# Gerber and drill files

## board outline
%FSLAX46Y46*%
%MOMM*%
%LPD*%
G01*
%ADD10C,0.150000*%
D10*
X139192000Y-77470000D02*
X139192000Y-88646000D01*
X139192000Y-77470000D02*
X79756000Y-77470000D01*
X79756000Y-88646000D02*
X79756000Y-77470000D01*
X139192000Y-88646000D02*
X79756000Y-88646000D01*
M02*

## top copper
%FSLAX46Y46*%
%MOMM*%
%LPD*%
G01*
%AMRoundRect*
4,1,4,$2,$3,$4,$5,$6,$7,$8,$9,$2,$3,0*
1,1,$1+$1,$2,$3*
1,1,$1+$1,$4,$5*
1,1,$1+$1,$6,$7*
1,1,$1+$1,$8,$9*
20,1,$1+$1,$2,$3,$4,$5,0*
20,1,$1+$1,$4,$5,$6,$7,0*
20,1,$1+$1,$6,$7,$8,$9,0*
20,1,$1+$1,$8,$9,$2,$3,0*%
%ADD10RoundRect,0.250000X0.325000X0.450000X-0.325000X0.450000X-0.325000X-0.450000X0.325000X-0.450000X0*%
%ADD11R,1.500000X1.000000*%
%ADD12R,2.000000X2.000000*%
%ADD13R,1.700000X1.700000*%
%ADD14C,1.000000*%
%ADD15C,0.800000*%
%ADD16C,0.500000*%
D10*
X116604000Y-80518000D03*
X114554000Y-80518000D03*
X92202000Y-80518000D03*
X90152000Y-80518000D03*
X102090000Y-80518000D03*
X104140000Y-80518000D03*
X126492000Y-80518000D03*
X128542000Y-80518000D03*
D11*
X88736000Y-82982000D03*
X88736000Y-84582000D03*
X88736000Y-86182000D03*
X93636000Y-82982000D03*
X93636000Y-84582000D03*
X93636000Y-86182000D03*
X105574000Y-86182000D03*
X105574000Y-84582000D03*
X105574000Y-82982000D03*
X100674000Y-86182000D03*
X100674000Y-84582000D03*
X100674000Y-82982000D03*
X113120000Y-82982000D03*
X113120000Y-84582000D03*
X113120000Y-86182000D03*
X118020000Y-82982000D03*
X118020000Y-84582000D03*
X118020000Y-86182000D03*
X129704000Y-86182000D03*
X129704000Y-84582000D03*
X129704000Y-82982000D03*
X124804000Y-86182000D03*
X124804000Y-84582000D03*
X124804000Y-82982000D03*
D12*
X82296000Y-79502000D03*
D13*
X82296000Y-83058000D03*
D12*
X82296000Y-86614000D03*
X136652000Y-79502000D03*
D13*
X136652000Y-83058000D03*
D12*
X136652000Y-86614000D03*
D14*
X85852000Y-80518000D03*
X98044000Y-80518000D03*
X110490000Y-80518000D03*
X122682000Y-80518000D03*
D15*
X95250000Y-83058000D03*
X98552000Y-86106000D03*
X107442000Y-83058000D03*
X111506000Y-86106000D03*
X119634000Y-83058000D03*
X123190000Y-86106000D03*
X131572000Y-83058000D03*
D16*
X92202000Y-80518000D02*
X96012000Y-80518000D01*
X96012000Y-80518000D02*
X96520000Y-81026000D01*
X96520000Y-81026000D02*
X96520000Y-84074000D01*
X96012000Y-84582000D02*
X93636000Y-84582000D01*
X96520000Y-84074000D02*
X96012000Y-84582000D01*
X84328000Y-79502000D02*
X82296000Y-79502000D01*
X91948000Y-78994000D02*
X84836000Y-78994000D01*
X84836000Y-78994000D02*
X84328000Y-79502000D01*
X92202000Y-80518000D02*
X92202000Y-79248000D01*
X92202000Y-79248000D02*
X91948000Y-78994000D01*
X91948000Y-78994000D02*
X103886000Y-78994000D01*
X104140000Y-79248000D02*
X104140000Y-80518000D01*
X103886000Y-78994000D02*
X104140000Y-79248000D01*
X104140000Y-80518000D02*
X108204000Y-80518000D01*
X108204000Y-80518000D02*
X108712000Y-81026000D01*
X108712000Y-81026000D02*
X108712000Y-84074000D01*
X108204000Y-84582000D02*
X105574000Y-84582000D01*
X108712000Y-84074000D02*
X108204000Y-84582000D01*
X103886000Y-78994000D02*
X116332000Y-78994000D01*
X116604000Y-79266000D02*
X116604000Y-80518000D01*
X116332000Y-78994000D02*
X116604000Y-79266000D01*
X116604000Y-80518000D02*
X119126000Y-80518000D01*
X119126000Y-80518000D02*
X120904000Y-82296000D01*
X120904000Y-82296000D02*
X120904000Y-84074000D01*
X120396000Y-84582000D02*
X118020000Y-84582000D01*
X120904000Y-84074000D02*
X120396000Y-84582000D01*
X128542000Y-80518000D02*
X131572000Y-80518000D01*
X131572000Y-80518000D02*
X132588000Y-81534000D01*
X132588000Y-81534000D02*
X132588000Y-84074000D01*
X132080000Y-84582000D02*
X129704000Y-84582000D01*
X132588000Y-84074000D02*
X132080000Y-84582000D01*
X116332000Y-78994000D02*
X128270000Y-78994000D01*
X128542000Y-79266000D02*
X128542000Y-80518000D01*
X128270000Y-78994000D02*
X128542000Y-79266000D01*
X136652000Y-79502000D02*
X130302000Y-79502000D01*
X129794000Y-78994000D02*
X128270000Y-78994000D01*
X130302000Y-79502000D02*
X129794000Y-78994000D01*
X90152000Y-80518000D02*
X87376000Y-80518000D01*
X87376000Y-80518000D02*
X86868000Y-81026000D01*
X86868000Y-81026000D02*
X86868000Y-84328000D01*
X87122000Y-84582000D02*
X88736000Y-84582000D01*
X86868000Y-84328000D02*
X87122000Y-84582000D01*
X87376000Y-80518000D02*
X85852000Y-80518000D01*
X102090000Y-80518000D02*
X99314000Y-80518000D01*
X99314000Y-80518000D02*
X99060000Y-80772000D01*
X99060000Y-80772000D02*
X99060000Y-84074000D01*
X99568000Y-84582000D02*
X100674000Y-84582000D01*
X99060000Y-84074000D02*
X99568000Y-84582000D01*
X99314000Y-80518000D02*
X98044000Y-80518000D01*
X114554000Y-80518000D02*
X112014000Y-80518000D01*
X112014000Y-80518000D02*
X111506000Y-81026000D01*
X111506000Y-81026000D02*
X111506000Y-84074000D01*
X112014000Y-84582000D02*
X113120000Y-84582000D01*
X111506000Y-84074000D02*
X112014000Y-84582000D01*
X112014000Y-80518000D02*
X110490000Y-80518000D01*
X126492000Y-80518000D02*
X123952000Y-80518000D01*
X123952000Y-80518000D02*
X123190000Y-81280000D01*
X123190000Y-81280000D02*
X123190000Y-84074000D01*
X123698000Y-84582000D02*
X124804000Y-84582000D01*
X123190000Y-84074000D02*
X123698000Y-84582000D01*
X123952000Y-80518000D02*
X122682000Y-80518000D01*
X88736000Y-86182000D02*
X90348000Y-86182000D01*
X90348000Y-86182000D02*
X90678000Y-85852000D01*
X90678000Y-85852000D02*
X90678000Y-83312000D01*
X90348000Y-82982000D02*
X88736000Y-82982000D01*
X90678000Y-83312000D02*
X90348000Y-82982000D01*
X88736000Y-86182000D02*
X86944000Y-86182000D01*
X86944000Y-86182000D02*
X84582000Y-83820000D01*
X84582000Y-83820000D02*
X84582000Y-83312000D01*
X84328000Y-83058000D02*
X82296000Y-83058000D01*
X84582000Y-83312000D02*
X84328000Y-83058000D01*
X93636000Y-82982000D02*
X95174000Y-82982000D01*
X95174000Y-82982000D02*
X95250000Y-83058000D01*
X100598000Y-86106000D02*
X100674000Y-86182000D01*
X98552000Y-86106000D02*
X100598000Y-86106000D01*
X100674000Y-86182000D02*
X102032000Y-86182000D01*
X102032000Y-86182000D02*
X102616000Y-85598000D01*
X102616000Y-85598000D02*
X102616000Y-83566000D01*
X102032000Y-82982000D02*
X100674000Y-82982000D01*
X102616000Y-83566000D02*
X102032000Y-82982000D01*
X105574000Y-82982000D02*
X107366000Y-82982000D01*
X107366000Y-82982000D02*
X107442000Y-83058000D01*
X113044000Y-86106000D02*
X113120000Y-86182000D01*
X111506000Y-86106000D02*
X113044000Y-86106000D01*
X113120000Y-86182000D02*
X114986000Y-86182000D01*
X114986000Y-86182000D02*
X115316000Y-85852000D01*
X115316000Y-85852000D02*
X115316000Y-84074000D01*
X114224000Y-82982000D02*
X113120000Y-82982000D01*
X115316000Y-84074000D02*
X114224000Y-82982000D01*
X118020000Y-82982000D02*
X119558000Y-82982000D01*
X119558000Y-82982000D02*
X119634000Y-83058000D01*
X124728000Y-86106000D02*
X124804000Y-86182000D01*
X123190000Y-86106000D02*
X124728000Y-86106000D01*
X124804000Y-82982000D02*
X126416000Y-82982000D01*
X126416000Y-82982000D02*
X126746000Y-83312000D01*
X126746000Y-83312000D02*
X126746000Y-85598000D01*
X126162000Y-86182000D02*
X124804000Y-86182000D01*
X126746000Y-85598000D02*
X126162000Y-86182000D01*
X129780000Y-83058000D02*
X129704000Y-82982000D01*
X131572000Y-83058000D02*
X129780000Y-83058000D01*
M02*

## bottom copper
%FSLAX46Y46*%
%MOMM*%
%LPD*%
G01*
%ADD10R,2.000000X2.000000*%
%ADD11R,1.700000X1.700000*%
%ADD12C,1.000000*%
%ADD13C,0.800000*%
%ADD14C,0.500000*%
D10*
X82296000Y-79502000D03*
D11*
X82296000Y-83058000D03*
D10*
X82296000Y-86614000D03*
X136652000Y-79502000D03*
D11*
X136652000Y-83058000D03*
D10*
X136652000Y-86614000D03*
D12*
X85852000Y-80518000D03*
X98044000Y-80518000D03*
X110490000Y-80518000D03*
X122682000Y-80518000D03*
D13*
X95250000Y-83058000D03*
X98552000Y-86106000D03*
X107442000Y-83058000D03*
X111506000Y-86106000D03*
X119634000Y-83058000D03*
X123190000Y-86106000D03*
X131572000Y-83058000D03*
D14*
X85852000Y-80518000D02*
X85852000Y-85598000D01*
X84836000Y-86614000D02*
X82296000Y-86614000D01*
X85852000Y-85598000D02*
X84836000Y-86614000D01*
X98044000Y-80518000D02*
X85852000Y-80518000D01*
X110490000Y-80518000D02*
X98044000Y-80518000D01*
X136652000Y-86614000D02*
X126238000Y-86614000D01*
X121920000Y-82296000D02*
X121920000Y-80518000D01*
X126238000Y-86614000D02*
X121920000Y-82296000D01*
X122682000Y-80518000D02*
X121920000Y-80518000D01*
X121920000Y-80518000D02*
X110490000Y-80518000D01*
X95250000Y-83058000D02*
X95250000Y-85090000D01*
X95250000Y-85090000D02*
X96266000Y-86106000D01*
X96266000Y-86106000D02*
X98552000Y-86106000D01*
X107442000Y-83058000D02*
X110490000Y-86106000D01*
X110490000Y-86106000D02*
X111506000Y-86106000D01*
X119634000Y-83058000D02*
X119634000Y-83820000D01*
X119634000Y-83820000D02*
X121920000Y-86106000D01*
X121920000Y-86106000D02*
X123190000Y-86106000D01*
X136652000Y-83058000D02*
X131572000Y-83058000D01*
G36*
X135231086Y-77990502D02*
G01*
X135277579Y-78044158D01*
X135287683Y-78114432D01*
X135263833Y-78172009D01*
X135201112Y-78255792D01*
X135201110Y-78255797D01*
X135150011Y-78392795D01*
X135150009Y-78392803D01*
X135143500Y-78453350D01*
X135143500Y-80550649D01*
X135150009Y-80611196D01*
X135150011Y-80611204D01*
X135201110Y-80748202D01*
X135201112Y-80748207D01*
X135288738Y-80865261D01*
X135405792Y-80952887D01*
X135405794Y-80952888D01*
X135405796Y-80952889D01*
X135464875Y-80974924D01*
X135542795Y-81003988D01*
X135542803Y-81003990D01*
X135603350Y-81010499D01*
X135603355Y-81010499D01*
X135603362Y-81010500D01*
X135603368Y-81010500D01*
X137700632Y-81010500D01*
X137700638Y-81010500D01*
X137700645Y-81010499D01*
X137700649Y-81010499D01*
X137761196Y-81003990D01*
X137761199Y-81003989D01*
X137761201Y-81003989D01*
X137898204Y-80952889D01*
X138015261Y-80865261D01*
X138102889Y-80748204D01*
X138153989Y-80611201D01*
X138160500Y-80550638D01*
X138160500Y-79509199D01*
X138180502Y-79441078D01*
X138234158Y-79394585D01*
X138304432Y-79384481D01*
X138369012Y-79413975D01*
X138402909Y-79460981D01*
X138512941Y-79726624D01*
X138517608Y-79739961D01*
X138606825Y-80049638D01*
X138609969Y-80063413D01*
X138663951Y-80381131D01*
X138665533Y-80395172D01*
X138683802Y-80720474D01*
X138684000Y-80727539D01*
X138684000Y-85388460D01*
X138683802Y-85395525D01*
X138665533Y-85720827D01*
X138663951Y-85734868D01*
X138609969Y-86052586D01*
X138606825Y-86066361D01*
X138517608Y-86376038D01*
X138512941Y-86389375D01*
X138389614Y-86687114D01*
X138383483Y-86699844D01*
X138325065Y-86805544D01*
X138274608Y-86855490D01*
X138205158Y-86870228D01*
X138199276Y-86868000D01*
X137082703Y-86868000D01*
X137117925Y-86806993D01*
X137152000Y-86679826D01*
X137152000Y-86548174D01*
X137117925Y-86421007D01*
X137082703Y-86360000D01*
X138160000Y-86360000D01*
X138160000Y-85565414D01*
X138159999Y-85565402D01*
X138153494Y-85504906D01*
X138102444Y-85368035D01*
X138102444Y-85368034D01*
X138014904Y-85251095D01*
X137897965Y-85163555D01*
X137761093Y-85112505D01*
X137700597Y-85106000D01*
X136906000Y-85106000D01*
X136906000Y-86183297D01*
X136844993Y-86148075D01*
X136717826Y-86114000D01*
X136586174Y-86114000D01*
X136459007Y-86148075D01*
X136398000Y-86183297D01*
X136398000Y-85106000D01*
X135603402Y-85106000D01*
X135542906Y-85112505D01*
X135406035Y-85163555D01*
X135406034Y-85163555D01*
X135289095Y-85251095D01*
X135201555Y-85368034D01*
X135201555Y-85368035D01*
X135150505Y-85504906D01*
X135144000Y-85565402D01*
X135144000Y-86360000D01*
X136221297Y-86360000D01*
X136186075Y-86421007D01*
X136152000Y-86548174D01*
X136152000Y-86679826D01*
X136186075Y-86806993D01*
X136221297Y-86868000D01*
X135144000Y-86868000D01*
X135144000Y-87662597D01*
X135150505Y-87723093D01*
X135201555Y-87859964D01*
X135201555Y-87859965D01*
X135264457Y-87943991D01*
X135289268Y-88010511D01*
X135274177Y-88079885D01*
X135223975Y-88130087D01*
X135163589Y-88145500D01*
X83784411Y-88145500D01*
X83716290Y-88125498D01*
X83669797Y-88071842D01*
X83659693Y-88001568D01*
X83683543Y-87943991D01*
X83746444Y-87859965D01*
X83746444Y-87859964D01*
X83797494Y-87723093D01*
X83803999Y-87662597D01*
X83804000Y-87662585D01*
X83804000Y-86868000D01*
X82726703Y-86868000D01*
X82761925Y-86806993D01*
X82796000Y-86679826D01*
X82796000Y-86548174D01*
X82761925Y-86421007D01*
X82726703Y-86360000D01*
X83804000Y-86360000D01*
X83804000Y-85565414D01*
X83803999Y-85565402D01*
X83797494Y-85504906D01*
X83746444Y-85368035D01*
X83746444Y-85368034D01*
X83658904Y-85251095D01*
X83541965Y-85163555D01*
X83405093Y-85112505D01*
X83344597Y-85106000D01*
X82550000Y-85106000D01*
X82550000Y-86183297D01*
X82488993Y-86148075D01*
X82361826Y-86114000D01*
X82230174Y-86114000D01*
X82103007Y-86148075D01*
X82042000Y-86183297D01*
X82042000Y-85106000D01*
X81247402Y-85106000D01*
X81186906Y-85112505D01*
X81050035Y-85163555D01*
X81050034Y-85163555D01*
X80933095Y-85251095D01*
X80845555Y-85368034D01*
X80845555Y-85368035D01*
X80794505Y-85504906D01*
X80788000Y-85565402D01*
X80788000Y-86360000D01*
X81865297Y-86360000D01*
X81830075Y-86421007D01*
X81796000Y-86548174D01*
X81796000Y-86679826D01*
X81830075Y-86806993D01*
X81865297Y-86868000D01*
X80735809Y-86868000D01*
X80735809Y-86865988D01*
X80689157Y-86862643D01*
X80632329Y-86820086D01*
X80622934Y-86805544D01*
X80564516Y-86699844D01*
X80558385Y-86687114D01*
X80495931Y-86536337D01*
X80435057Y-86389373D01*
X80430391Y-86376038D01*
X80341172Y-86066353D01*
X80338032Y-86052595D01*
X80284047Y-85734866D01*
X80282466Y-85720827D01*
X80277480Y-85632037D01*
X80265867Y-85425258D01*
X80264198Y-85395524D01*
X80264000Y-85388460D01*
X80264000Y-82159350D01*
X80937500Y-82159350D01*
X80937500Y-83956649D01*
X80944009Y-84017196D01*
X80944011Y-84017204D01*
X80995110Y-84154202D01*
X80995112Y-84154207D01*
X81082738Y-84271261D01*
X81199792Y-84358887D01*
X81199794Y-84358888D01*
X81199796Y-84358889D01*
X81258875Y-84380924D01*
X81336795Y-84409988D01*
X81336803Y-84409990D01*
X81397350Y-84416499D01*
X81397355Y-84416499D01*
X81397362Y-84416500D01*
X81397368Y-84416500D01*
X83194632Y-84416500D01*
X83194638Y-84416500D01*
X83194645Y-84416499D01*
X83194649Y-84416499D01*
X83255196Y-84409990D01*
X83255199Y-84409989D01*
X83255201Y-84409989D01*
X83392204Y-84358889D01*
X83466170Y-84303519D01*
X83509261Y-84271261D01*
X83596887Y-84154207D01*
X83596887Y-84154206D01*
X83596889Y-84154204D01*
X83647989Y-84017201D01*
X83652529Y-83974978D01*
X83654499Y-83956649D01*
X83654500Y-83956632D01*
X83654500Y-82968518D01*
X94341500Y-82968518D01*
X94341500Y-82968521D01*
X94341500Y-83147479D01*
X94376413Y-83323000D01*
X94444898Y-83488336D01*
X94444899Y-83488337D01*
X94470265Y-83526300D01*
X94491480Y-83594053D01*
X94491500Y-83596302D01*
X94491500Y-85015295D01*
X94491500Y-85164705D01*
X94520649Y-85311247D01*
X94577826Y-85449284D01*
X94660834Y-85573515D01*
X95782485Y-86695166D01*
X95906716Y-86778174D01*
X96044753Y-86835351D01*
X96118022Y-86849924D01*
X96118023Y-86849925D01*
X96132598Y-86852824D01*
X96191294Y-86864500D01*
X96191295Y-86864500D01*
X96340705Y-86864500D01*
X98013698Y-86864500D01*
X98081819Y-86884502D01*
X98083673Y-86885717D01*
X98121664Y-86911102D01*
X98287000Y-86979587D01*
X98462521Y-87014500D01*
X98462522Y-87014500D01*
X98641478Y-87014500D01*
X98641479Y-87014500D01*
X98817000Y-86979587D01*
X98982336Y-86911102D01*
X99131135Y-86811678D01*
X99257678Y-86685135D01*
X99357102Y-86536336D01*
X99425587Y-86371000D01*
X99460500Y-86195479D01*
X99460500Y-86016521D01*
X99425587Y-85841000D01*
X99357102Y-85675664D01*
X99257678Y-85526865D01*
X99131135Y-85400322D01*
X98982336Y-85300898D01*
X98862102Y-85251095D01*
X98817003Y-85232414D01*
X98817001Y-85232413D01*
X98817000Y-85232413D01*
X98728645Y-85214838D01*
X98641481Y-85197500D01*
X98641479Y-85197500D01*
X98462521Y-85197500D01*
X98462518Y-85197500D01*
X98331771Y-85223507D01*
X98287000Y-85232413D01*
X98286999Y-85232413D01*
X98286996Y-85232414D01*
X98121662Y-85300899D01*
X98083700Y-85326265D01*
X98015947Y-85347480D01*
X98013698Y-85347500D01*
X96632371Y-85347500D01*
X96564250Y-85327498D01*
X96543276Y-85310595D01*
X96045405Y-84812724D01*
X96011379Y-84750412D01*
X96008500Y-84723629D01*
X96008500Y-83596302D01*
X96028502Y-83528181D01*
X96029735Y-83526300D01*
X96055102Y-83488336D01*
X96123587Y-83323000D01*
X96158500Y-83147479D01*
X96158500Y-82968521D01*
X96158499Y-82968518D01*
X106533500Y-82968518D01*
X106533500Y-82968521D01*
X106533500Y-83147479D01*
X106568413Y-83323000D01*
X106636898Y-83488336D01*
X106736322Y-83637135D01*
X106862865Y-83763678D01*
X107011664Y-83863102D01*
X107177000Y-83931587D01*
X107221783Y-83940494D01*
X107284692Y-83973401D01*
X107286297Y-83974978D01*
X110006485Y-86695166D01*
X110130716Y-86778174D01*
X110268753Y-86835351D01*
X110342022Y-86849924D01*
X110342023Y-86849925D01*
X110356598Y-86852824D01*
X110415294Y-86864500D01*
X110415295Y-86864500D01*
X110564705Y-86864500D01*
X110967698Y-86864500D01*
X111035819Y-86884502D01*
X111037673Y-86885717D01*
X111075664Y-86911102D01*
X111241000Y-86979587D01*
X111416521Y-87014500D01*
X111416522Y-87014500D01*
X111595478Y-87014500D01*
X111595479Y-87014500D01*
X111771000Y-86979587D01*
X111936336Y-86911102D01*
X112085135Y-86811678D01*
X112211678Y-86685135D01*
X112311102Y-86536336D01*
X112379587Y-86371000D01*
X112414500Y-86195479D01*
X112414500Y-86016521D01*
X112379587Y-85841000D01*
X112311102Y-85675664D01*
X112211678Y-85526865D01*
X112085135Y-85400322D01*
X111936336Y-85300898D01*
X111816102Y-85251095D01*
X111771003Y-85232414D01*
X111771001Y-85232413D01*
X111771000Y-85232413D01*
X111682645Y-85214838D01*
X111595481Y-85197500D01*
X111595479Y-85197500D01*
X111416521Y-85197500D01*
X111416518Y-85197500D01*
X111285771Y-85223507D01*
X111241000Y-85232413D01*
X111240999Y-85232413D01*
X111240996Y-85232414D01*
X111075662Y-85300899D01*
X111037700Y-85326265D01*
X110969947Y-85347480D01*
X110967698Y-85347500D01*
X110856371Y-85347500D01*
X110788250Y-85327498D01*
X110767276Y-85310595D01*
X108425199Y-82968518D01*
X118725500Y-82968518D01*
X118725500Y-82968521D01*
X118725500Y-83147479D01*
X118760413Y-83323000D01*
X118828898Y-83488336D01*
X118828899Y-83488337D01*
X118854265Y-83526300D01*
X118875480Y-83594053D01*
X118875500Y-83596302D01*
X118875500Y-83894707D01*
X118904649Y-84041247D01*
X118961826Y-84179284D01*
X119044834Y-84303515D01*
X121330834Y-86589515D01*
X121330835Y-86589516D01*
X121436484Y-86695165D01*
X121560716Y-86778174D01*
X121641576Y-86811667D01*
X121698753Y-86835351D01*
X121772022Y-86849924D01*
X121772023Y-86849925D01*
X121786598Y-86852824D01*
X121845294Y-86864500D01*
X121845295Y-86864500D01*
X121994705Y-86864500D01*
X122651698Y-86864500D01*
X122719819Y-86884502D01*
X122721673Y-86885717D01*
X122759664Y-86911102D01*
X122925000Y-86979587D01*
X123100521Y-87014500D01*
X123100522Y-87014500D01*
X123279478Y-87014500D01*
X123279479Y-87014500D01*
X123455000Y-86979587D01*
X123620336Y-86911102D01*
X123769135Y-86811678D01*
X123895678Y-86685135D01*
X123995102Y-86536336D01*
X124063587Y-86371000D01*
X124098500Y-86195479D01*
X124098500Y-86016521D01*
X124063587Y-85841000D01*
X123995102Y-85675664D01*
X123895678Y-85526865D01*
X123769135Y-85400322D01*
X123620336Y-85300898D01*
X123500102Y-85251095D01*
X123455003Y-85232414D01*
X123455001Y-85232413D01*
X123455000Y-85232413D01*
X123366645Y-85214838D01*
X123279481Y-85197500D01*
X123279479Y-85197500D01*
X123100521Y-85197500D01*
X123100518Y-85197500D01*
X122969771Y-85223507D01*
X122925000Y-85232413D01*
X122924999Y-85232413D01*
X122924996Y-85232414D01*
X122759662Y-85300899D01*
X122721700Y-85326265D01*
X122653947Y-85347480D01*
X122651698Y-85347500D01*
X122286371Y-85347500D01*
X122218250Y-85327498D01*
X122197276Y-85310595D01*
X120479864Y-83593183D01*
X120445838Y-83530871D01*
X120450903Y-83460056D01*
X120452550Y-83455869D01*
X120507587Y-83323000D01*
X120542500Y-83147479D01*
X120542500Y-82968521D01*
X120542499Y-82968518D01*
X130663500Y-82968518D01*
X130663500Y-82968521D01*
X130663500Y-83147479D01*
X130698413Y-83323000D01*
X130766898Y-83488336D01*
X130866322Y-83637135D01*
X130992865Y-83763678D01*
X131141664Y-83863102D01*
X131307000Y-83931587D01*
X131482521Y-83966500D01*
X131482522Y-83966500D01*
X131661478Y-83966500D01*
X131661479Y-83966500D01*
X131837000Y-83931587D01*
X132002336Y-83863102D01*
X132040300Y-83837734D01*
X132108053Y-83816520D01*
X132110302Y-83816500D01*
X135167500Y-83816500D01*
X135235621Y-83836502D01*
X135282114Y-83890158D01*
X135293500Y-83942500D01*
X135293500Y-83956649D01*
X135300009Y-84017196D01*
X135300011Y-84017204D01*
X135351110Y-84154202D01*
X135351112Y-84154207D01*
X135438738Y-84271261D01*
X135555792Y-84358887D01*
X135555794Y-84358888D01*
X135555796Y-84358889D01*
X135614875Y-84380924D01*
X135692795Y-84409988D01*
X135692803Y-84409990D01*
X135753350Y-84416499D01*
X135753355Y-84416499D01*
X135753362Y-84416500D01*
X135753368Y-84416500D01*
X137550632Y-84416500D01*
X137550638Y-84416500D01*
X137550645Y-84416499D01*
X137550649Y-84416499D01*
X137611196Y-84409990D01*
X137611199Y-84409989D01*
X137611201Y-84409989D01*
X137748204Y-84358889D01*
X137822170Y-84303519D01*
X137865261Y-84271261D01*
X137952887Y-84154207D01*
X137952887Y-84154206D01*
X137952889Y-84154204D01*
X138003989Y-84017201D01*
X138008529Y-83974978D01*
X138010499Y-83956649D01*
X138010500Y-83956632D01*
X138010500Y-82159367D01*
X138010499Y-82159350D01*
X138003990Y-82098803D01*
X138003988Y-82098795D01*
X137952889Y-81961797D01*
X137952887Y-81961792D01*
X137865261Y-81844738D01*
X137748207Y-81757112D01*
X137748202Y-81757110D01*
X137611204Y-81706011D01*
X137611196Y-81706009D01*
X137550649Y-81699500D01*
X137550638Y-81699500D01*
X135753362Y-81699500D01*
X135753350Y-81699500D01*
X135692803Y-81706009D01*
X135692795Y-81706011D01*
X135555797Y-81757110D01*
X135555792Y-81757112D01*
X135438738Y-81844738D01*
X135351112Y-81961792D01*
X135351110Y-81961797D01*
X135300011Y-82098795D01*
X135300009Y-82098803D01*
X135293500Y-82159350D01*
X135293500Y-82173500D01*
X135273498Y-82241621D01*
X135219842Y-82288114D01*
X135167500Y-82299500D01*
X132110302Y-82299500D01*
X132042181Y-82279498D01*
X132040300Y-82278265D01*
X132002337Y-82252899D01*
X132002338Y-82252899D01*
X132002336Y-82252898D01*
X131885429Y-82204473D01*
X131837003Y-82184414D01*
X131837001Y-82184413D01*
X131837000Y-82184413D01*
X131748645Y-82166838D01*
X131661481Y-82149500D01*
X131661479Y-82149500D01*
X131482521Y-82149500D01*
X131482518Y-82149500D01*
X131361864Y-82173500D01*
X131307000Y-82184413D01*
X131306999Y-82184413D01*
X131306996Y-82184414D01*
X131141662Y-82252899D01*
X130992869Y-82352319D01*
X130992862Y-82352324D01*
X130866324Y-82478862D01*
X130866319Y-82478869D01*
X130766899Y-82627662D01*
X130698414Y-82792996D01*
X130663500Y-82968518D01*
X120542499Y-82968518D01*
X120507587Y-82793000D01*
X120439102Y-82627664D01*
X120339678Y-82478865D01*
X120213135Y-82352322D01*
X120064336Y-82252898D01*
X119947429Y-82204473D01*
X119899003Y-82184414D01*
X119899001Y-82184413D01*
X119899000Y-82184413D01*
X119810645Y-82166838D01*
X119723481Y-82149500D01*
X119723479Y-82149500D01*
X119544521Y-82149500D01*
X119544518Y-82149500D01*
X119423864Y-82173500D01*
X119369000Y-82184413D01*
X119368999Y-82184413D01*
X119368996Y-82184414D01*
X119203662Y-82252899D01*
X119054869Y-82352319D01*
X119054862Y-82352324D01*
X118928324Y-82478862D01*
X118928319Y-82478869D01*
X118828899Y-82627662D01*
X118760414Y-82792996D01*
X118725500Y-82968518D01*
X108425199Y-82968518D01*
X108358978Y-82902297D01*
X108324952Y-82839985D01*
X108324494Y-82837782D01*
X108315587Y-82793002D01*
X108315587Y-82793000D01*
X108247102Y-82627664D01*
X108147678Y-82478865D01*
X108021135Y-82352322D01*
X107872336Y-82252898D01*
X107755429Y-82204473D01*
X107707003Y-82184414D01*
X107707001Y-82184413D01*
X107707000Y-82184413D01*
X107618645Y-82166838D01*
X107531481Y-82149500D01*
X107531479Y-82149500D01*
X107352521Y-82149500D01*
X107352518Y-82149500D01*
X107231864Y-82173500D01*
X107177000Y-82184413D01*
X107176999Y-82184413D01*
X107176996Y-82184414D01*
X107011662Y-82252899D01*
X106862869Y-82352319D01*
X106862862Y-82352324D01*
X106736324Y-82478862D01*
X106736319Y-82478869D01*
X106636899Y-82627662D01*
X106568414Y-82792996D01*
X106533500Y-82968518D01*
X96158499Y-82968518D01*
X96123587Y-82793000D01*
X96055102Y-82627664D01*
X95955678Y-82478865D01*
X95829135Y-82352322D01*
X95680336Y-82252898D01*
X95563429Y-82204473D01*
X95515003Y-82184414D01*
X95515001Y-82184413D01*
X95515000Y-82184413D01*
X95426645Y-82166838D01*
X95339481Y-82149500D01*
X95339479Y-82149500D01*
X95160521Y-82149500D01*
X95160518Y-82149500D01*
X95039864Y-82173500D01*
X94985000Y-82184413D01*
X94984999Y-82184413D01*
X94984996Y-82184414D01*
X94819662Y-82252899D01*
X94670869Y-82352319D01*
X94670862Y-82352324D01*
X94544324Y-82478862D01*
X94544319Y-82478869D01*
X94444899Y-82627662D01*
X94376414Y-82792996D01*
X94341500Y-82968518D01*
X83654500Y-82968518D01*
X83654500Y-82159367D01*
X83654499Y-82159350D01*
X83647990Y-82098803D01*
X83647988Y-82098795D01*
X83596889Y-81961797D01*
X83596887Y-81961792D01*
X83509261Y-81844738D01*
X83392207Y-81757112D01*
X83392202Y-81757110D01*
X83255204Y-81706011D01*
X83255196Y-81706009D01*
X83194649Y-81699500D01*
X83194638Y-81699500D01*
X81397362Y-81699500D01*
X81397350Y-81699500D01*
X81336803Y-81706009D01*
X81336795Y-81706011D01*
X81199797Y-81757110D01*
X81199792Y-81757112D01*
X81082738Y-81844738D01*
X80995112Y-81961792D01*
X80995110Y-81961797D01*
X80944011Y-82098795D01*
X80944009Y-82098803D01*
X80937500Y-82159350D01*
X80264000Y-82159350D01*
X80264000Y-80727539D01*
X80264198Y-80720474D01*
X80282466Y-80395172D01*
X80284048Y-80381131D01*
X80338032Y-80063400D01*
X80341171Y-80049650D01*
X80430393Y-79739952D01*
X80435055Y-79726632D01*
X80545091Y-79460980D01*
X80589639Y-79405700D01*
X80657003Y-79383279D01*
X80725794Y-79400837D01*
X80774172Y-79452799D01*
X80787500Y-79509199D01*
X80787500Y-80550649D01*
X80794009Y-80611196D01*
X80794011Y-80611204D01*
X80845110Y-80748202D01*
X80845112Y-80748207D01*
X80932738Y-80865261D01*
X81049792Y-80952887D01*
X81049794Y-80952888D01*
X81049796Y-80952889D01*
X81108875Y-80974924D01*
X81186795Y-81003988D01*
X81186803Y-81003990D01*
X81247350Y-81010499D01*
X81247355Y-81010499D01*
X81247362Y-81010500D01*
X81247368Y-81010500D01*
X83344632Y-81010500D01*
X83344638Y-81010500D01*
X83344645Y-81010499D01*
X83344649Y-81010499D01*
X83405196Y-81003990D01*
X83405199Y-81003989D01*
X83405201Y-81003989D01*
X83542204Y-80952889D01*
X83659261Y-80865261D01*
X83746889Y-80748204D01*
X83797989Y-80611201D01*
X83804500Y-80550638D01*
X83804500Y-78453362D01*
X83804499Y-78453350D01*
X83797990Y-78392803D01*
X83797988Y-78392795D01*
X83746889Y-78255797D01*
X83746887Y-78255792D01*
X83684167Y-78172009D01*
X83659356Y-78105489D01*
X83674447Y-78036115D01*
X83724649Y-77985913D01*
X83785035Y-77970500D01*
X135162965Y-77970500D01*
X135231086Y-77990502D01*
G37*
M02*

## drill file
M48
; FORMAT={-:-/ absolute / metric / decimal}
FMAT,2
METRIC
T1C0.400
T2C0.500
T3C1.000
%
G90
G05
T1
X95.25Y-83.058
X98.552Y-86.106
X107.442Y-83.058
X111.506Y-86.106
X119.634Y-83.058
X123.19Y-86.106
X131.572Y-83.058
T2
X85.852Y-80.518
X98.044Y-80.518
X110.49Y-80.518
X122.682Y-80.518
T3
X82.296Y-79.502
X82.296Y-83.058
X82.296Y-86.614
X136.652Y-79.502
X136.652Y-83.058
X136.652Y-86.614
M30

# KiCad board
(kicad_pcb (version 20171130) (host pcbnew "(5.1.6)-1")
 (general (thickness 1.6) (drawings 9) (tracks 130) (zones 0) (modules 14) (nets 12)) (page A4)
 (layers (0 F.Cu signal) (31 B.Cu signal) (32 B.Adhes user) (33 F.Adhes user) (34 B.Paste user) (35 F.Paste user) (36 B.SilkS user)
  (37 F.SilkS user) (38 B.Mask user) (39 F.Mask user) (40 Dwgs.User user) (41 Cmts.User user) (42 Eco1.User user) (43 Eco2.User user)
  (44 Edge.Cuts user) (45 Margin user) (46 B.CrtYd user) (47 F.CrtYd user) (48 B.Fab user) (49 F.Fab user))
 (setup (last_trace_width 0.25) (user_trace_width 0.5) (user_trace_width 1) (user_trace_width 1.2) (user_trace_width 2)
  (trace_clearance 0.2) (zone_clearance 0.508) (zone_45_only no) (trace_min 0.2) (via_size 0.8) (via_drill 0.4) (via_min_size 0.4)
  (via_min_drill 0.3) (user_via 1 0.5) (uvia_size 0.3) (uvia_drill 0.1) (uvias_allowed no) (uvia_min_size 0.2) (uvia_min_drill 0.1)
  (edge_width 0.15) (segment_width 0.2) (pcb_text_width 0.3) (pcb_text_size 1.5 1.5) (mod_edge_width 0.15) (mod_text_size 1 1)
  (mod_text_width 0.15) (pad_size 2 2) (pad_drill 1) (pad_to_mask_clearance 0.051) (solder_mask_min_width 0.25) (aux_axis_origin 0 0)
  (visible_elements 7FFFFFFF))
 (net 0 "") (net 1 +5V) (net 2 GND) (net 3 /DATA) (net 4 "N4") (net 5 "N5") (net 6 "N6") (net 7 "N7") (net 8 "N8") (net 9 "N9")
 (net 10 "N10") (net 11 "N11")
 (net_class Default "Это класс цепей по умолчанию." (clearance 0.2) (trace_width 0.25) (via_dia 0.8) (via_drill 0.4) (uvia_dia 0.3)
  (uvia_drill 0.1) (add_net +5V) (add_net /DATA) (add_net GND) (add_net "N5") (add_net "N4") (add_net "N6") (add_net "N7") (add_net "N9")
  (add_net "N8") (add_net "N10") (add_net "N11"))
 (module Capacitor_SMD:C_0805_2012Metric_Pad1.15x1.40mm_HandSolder (layer F.Cu) (at 115.579 80.518 180)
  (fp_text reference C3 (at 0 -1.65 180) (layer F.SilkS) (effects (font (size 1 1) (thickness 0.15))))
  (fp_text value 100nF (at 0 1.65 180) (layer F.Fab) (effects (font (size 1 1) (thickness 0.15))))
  (pad 1 smd roundrect (at -1.025 0 180) (size 1.15 1.4) (layers F.Cu F.Paste F.Mask) (roundrect_rratio 0.217391) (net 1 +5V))
  (pad 2 smd roundrect (at 1.025 0 180) (size 1.15 1.4) (layers F.Cu F.Paste F.Mask) (roundrect_rratio 0.217391) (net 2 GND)))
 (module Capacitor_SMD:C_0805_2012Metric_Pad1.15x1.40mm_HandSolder (layer F.Cu) (at 91.177 80.518 180)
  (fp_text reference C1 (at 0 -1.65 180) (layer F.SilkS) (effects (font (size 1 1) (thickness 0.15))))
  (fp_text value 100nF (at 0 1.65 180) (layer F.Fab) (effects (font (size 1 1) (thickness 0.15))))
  (pad 1 smd roundrect (at -1.025 0 180) (size 1.15 1.4) (layers F.Cu F.Paste F.Mask) (roundrect_rratio 0.217391) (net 1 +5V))
  (pad 2 smd roundrect (at 1.025 0 180) (size 1.15 1.4) (layers F.Cu F.Paste F.Mask) (roundrect_rratio 0.217391) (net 2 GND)))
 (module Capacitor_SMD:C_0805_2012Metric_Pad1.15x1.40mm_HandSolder (layer F.Cu) (at 103.115 80.518 180)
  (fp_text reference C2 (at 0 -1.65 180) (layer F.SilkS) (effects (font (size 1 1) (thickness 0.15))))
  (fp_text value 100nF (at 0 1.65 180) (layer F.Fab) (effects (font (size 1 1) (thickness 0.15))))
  (pad 2 smd roundrect (at 1.025 0 180) (size 1.15 1.4) (layers F.Cu F.Paste F.Mask) (roundrect_rratio 0.217391) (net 2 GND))
  (pad 1 smd roundrect (at -1.025 0 180) (size 1.15 1.4) (layers F.Cu F.Paste F.Mask) (roundrect_rratio 0.217391) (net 1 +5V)))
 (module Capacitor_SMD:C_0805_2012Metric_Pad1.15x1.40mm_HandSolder (layer F.Cu) (at 127.517 80.518 180)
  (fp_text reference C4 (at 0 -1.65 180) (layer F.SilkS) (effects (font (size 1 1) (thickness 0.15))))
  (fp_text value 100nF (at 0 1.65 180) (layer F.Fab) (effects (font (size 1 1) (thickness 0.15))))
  (pad 2 smd roundrect (at 1.025 0 180) (size 1.15 1.4) (layers F.Cu F.Paste F.Mask) (roundrect_rratio 0.217391) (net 2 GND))
  (pad 1 smd roundrect (at -1.025 0 180) (size 1.15 1.4) (layers F.Cu F.Paste F.Mask) (roundrect_rratio 0.217391) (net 1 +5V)))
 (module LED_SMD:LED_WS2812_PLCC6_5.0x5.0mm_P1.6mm (layer F.Cu) (at 91.186 84.582 180)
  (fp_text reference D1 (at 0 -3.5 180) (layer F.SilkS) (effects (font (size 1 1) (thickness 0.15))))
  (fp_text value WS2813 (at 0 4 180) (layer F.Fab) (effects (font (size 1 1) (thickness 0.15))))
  (pad 4 smd rect (at 2.45 1.6 180) (size 1.5 1) (layers F.Cu F.Paste F.Mask) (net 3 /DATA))
  (pad 5 smd rect (at 2.45 0 180) (size 1.5 1) (layers F.Cu F.Paste F.Mask) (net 2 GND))
  (pad 6 smd rect (at 2.45 -1.6 180) (size 1.5 1) (layers F.Cu F.Paste F.Mask) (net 3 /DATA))
  (pad 3 smd rect (at -2.45 1.6 180) (size 1.5 1) (layers F.Cu F.Paste F.Mask) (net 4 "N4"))
  (pad 2 smd rect (at -2.45 0 180) (size 1.5 1) (layers F.Cu F.Paste F.Mask) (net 1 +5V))
  (pad 1 smd rect (at -2.45 -1.6 180) (size 1.5 1) (layers F.Cu F.Paste F.Mask) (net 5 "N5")))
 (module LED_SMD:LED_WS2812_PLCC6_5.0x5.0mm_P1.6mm (layer F.Cu) (at 103.124 84.582 180)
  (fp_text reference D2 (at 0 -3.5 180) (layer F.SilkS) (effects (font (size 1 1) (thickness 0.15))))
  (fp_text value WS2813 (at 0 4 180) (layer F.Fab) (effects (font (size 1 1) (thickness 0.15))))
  (pad 1 smd rect (at -2.45 -1.6 180) (size 1.5 1) (layers F.Cu F.Paste F.Mask) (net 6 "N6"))
  (pad 2 smd rect (at -2.45 0 180) (size 1.5 1) (layers F.Cu F.Paste F.Mask) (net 1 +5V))
  (pad 3 smd rect (at -2.45 1.6 180) (size 1.5 1) (layers F.Cu F.Paste F.Mask) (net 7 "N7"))
  (pad 6 smd rect (at 2.45 -1.6 180) (size 1.5 1) (layers F.Cu F.Paste F.Mask) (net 4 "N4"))
  (pad 5 smd rect (at 2.45 0 180) (size 1.5 1) (layers F.Cu F.Paste F.Mask) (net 2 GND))
  (pad 4 smd rect (at 2.45 1.6 180) (size 1.5 1) (layers F.Cu F.Paste F.Mask) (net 4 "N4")))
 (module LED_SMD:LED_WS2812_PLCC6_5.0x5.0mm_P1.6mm (layer F.Cu) (at 115.57 84.582 180)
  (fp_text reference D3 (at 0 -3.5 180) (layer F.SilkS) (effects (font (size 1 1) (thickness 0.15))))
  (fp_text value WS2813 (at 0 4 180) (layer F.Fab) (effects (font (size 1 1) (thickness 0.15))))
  (pad 4 smd rect (at 2.45 1.6 180) (size 1.5 1) (layers F.Cu F.Paste F.Mask) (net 7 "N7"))
  (pad 5 smd rect (at 2.45 0 180) (size 1.5 1) (layers F.Cu F.Paste F.Mask) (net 2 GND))
  (pad 6 smd rect (at 2.45 -1.6 180) (size 1.5 1) (layers F.Cu F.Paste F.Mask) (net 7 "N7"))
  (pad 3 smd rect (at -2.45 1.6 180) (size 1.5 1) (layers F.Cu F.Paste F.Mask) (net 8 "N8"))
  (pad 2 smd rect (at -2.45 0 180) (size 1.5 1) (layers F.Cu F.Paste F.Mask) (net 1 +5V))
  (pad 1 smd rect (at -2.45 -1.6 180) (size 1.5 1) (layers F.Cu F.Paste F.Mask) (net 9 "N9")))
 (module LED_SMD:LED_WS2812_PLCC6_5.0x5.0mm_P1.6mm (layer F.Cu) (at 127.254 84.582 180)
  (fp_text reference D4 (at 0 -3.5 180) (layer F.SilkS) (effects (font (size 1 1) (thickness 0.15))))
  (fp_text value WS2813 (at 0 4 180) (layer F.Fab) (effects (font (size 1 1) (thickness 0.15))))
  (pad 1 smd rect (at -2.45 -1.6 180) (size 1.5 1) (layers F.Cu F.Paste F.Mask) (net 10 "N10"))
  (pad 2 smd rect (at -2.45 0 180) (size 1.5 1) (layers F.Cu F.Paste F.Mask) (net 1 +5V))
  (pad 3 smd rect (at -2.45 1.6 180) (size 1.5 1) (layers F.Cu F.Paste F.Mask) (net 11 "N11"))
  (pad 6 smd rect (at 2.45 -1.6 180) (size 1.5 1) (layers F.Cu F.Paste F.Mask) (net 8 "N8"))
  (pad 5 smd rect (at 2.45 0 180) (size 1.5 1) (layers F.Cu F.Paste F.Mask) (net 2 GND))
  (pad 4 smd rect (at 2.45 1.6 180) (size 1.5 1) (layers F.Cu F.Paste F.Mask) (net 8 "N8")))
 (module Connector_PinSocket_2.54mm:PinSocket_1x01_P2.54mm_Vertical (layer F.Cu) (at 82.296 79.502)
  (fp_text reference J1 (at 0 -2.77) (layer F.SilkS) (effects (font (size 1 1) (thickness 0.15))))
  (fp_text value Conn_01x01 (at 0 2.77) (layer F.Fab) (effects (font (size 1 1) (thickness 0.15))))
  (pad 1 thru_hole rect (at 0 0) (size 2 2) (drill 1) (layers *.Cu *.Mask) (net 1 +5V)))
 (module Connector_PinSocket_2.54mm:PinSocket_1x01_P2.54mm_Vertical (layer F.Cu) (at 82.296 83.058)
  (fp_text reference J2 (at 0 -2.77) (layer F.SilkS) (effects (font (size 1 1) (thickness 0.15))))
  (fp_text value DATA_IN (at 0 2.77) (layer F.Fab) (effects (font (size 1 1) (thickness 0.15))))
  (pad 1 thru_hole rect (at 0 0) (size 1.7 1.7) (drill 1) (layers *.Cu *.Mask) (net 3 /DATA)))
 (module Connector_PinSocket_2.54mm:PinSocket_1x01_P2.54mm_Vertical (layer F.Cu) (at 82.296 86.614)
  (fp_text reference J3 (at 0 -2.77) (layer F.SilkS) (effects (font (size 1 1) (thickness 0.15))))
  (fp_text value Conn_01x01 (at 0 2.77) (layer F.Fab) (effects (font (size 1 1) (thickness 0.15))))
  (pad 1 thru_hole rect (at 0 0) (size 2 2) (drill 1) (layers *.Cu *.Mask) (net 2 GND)))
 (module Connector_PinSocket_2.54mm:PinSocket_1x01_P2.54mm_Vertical (layer F.Cu) (at 136.652 79.502)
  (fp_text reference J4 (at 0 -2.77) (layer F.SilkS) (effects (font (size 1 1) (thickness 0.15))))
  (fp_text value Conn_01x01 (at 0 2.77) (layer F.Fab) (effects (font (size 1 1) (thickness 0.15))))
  (pad 1 thru_hole rect (at 0 0) (size 2 2) (drill 1) (layers *.Cu *.Mask) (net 1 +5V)))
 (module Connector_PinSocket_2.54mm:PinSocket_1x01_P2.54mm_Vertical (layer F.Cu) (at 136.652 83.058)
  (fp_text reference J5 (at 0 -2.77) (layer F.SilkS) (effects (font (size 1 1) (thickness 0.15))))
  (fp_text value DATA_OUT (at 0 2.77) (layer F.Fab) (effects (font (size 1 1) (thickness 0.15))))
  (pad 1 thru_hole rect (at 0 0) (size 1.7 1.7) (drill 1) (layers *.Cu *.Mask) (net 11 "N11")))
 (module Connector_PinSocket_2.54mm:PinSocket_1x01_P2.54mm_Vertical (layer F.Cu) (at 136.652 86.614)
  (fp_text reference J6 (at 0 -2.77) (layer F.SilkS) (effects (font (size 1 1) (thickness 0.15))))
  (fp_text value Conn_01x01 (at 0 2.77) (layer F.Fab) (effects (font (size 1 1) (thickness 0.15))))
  (pad 1 thru_hole rect (at 0 0) (size 2 2) (drill 1) (layers *.Cu *.Mask) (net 2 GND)))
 (gr_line (start 139.192 77.47) (end 139.192 88.646) (layer Edge.Cuts) (width 0.15))
 (gr_line (start 139.192 77.47) (end 79.756 77.47) (layer Edge.Cuts) (width 0.15))
 (gr_line (start 79.756 88.646) (end 79.756 77.47) (layer Edge.Cuts) (width 0.15))
 (gr_line (start 139.192 88.646) (end 79.756 88.646) (layer Edge.Cuts) (width 0.15))
 (segment (start 92.202 80.518) (end 96.012 80.518) (width 0.5) (layer F.Cu) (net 1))
 (segment (start 96.012 80.518) (end 96.52 81.026) (width 0.5) (layer F.Cu) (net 1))
 (segment (start 96.52 81.026) (end 96.52 84.074) (width 0.5) (layer F.Cu) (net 1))
 (segment (start 96.012 84.582) (end 93.636 84.582) (width 0.5) (layer F.Cu) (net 1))
 (segment (start 96.52 84.074) (end 96.012 84.582) (width 0.5) (layer F.Cu) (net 1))
 (segment (start 84.328 79.502) (end 82.296 79.502) (width 0.5) (layer F.Cu) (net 1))
 (segment (start 91.948 78.994) (end 84.836 78.994) (width 0.5) (layer F.Cu) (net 1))
 (segment (start 84.836 78.994) (end 84.328 79.502) (width 0.5) (layer F.Cu) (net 1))
 (segment (start 92.202 80.518) (end 92.202 79.248) (width 0.5) (layer F.Cu) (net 1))
 (segment (start 92.202 79.248) (end 91.948 78.994) (width 0.5) (layer F.Cu) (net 1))
 (segment (start 91.948 78.994) (end 103.886 78.994) (width 0.5) (layer F.Cu) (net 1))
 (segment (start 104.14 79.248) (end 104.14 80.518) (width 0.5) (layer F.Cu) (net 1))
 (segment (start 103.886 78.994) (end 104.14 79.248) (width 0.5) (layer F.Cu) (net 1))
 (segment (start 104.14 80.518) (end 108.204 80.518) (width 0.5) (layer F.Cu) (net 1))
 (segment (start 108.204 80.518) (end 108.712 81.026) (width 0.5) (layer F.Cu) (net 1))
 (segment (start 108.712 81.026) (end 108.712 84.074) (width 0.5) (layer F.Cu) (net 1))
 (segment (start 108.204 84.582) (end 105.574 84.582) (width 0.5) (layer F.Cu) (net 1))
 (segment (start 108.712 84.074) (end 108.204 84.582) (width 0.5) (layer F.Cu) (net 1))
 (segment (start 103.886 78.994) (end 116.332 78.994) (width 0.5) (layer F.Cu) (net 1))
 (segment (start 116.604 79.266) (end 116.604 80.518) (width 0.5) (layer F.Cu) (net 1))
 (segment (start 116.332 78.994) (end 116.604 79.266) (width 0.5) (layer F.Cu) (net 1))
 (segment (start 116.604 80.518) (end 119.126 80.518) (width 0.5) (layer F.Cu) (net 1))
 (segment (start 119.126 80.518) (end 120.904 82.296) (width 0.5) (layer F.Cu) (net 1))
 (segment (start 120.904 82.296) (end 120.904 84.074) (width 0.5) (layer F.Cu) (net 1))
 (segment (start 120.396 84.582) (end 118.02 84.582) (width 0.5) (layer F.Cu) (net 1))
 (segment (start 120.904 84.074) (end 120.396 84.582) (width 0.5) (layer F.Cu) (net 1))
 (segment (start 128.542 80.518) (end 131.572 80.518) (width 0.5) (layer F.Cu) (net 1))
 (segment (start 131.572 80.518) (end 132.588 81.534) (width 0.5) (layer F.Cu) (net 1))
 (segment (start 132.588 81.534) (end 132.588 84.074) (width 0.5) (layer F.Cu) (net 1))
 (segment (start 132.08 84.582) (end 129.704 84.582) (width 0.5) (layer F.Cu) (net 1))
 (segment (start 132.588 84.074) (end 132.08 84.582) (width 0.5) (layer F.Cu) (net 1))
 (segment (start 116.332 78.994) (end 128.27 78.994) (width 0.5) (layer F.Cu) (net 1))
 (segment (start 128.542 79.266) (end 128.542 80.518) (width 0.5) (layer F.Cu) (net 1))
 (segment (start 128.27 78.994) (end 128.542 79.266) (width 0.5) (layer F.Cu) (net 1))
 (segment (start 136.652 79.502) (end 130.302 79.502) (width 0.5) (layer F.Cu) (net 1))
 (segment (start 129.794 78.994) (end 128.27 78.994) (width 0.5) (layer F.Cu) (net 1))
 (segment (start 130.302 79.502) (end 129.794 78.994) (width 0.5) (layer F.Cu) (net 1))
 (segment (start 90.152 80.518) (end 87.376 80.518) (width 0.5) (layer F.Cu) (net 2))
 (segment (start 87.376 80.518) (end 86.868 81.026) (width 0.5) (layer F.Cu) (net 2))
 (segment (start 86.868 81.026) (end 86.868 84.328) (width 0.5) (layer F.Cu) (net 2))
 (segment (start 87.122 84.582) (end 88.736 84.582) (width 0.5) (layer F.Cu) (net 2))
 (segment (start 86.868 84.328) (end 87.122 84.582) (width 0.5) (layer F.Cu) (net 2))
 (via (at 85.852 80.518) (size 1) (drill 0.5) (layers F.Cu B.Cu) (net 2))
 (segment (start 87.376 80.518) (end 85.852 80.518) (width 0.5) (layer F.Cu) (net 2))
 (segment (start 85.852 80.518) (end 85.852 85.598) (width 0.5) (layer B.Cu) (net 2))
 (segment (start 84.836 86.614) (end 82.296 86.614) (width 0.5) (layer B.Cu) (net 2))
 (segment (start 85.852 85.598) (end 84.836 86.614) (width 0.5) (layer B.Cu) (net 2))
 (segment (start 102.09 80.518) (end 99.314 80.518) (width 0.5) (layer F.Cu) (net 2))
 (segment (start 99.314 80.518) (end 99.06 80.772) (width 0.5) (layer F.Cu) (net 2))
 (segment (start 99.06 80.772) (end 99.06 84.074) (width 0.5) (layer F.Cu) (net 2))
 (segment (start 99.568 84.582) (end 100.674 84.582) (width 0.5) (layer F.Cu) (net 2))
 (segment (start 99.06 84.074) (end 99.568 84.582) (width 0.5) (layer F.Cu) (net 2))
 (via (at 98.044 80.518) (size 1) (drill 0.5) (layers F.Cu B.Cu) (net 2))
 (segment (start 99.314 80.518) (end 98.044 80.518) (width 0.5) (layer F.Cu) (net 2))
 (segment (start 98.044 80.518) (end 85.852 80.518) (width 0.5) (layer B.Cu) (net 2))
 (segment (start 114.554 80.518) (end 112.014 80.518) (width 0.5) (layer F.Cu) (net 2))
 (segment (start 112.014 80.518) (end 111.506 81.026) (width 0.5) (layer F.Cu) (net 2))
 (segment (start 111.506 81.026) (end 111.506 84.074) (width 0.5) (layer F.Cu) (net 2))
 (segment (start 112.014 84.582) (end 113.12 84.582) (width 0.5) (layer F.Cu) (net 2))
 (segment (start 111.506 84.074) (end 112.014 84.582) (width 0.5) (layer F.Cu) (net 2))
 (via (at 110.49 80.518) (size 1) (drill 0.5) (layers F.Cu B.Cu) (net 2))
 (segment (start 112.014 80.518) (end 110.49 80.518) (width 0.5) (layer F.Cu) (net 2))
 (segment (start 110.49 80.518) (end 98.044 80.518) (width 0.5) (layer B.Cu) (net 2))
 (segment (start 126.492 80.518) (end 123.952 80.518) (width 0.5) (layer F.Cu) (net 2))
 (segment (start 123.952 80.518) (end 123.19 81.28) (width 0.5) (layer F.Cu) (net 2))
 (segment (start 123.19 81.28) (end 123.19 84.074) (width 0.5) (layer F.Cu) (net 2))
 (segment (start 123.698 84.582) (end 124.804 84.582) (width 0.5) (layer F.Cu) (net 2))
 (segment (start 123.19 84.074) (end 123.698 84.582) (width 0.5) (layer F.Cu) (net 2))
 (via (at 122.682 80.518) (size 1) (drill 0.5) (layers F.Cu B.Cu) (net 2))
 (segment (start 123.952 80.518) (end 122.682 80.518) (width 0.5) (layer F.Cu) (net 2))
 (segment (start 136.652 86.614) (end 126.238 86.614) (width 0.5) (layer B.Cu) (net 2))
 (segment (start 121.92 82.296) (end 121.92 80.518) (width 0.5) (layer B.Cu) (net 2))
 (segment (start 126.238 86.614) (end 121.92 82.296) (width 0.5) (layer B.Cu) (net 2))
 (segment (start 122.682 80.518) (end 121.92 80.518) (width 0.5) (layer B.Cu) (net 2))
 (segment (start 121.92 80.518) (end 110.49 80.518) (width 0.5) (layer B.Cu) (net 2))
 (segment (start 88.736 86.182) (end 90.348 86.182) (width 0.5) (layer F.Cu) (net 3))
 (segment (start 90.348 86.182) (end 90.678 85.852) (width 0.5) (layer F.Cu) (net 3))
 (segment (start 90.678 85.852) (end 90.678 83.312) (width 0.5) (layer F.Cu) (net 3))
 (segment (start 90.348 82.982) (end 88.736 82.982) (width 0.5) (layer F.Cu) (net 3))
 (segment (start 90.678 83.312) (end 90.348 82.982) (width 0.5) (layer F.Cu) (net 3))
 (segment (start 88.736 86.182) (end 86.944 86.182) (width 0.5) (layer F.Cu) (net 3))
 (segment (start 86.944 86.182) (end 84.582 83.82) (width 0.5) (layer F.Cu) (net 3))
 (segment (start 84.582 83.82) (end 84.582 83.312) (width 0.5) (layer F.Cu) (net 3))
 (segment (start 84.328 83.058) (end 82.296 83.058) (width 0.5) (layer F.Cu) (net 3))
 (segment (start 84.582 83.312) (end 84.328 83.058) (width 0.5) (layer F.Cu) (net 3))
 (via (at 95.25 83.058) (size 0.8) (drill 0.4) (layers F.Cu B.Cu) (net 4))
 (segment (start 93.636 82.982) (end 95.174 82.982) (width 0.5) (layer F.Cu) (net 4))
 (segment (start 95.174 82.982) (end 95.25 83.058) (width 0.5) (layer F.Cu) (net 4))
 (segment (start 95.25 83.058) (end 95.25 85.09) (width 0.5) (layer B.Cu) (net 4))
 (via (at 98.552 86.106) (size 0.8) (drill 0.4) (layers F.Cu B.Cu) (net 4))
 (segment (start 95.25 85.09) (end 96.266 86.106) (width 0.5) (layer B.Cu) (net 4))
 (segment (start 96.266 86.106) (end 98.552 86.106) (width 0.5) (layer B.Cu) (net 4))
 (segment (start 100.598 86.106) (end 100.674 86.182) (width 0.5) (layer F.Cu) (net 4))
 (segment (start 98.552 86.106) (end 100.598 86.106) (width 0.5) (layer F.Cu) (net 4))
 (segment (start 100.674 86.182) (end 102.032 86.182) (width 0.5) (layer F.Cu) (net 4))
 (segment (start 102.032 86.182) (end 102.616 85.598) (width 0.5) (layer F.Cu) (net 4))
 (segment (start 102.616 85.598) (end 102.616 83.566) (width 0.5) (layer F.Cu) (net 4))
 (segment (start 102.032 82.982) (end 100.674 82.982) (width 0.5) (layer F.Cu) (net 4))
 (segment (start 102.616 83.566) (end 102.032 82.982) (width 0.5) (layer F.Cu) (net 4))
 (via (at 107.442 83.058) (size 0.8) (drill 0.4) (layers F.Cu B.Cu) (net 7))
 (segment (start 105.574 82.982) (end 107.366 82.982) (width 0.5) (layer F.Cu) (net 7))
 (segment (start 107.366 82.982) (end 107.442 83.058) (width 0.5) (layer F.Cu) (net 7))
 (via (at 111.506 86.106) (size 0.8) (drill 0.4) (layers F.Cu B.Cu) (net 7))
 (segment (start 107.442 83.058) (end 110.49 86.106) (width 0.5) (layer B.Cu) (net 7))
 (segment (start 110.49 86.106) (end 111.506 86.106) (width 0.5) (layer B.Cu) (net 7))
 (segment (start 113.044 86.106) (end 113.12 86.182) (width 0.5) (layer F.Cu) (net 7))
 (segment (start 111.506 86.106) (end 113.044 86.106) (width 0.5) (layer F.Cu) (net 7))
 (segment (start 113.12 86.182) (end 114.986 86.182) (width 0.5) (layer F.Cu) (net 7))
 (segment (start 114.986 86.182) (end 115.316 85.852) (width 0.5) (layer F.Cu) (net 7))
 (segment (start 115.316 85.852) (end 115.316 84.074) (width 0.5) (layer F.Cu) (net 7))
 (segment (start 114.224 82.982) (end 113.12 82.982) (width 0.5) (layer F.Cu) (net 7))
 (segment (start 115.316 84.074) (end 114.224 82.982) (width 0.5) (layer F.Cu) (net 7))
 (via (at 119.634 83.058) (size 0.8) (drill 0.4) (layers F.Cu B.Cu) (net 8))
 (segment (start 118.02 82.982) (end 119.558 82.982) (width 0.5) (layer F.Cu) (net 8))
 (segment (start 119.558 82.982) (end 119.634 83.058) (width 0.5) (layer F.Cu) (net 8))
 (segment (start 119.634 83.058) (end 119.634 83.82) (width 0.5) (layer B.Cu) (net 8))
 (segment (start 119.634 83.82) (end 121.92 86.106) (width 0.5) (layer B.Cu) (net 8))
 (via (at 123.19 86.106) (size 0.8) (drill 0.4) (layers F.Cu B.Cu) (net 8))
 (segment (start 121.92 86.106) (end 123.19 86.106) (width 0.5) (layer B.Cu) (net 8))
 (segment (start 124.728 86.106) (end 124.804 86.182) (width 0.5) (layer F.Cu) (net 8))
 (segment (start 123.19 86.106) (end 124.728 86.106) (width 0.5) (layer F.Cu) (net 8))
 (segment (start 124.804 82.982) (end 126.416 82.982) (width 0.5) (layer F.Cu) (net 8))
 (segment (start 126.416 82.982) (end 126.746 83.312) (width 0.5) (layer F.Cu) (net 8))
 (segment (start 126.746 83.312) (end 126.746 85.598) (width 0.5) (layer F.Cu) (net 8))
 (segment (start 126.162 86.182) (end 124.804 86.182) (width 0.5) (layer F.Cu) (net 8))
 (segment (start 126.746 85.598) (end 126.162 86.182) (width 0.5) (layer F.Cu) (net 8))
 (via (at 131.572 83.058) (size 0.8) (drill 0.4) (layers F.Cu B.Cu) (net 11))
 (segment (start 136.652 83.058) (end 131.572 83.058) (width 0.5) (layer B.Cu) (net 11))
 (segment (start 129.78 83.058) (end 129.704 82.982) (width 0.5) (layer F.Cu) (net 11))
 (segment (start 131.572 83.058) (end 129.78 83.058) (width 0.5) (layer F.Cu) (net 11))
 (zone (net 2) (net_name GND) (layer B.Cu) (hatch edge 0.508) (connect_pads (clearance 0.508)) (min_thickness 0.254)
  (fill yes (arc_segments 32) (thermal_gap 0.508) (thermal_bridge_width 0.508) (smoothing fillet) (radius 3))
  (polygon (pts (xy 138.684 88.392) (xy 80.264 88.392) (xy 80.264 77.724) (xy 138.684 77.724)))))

